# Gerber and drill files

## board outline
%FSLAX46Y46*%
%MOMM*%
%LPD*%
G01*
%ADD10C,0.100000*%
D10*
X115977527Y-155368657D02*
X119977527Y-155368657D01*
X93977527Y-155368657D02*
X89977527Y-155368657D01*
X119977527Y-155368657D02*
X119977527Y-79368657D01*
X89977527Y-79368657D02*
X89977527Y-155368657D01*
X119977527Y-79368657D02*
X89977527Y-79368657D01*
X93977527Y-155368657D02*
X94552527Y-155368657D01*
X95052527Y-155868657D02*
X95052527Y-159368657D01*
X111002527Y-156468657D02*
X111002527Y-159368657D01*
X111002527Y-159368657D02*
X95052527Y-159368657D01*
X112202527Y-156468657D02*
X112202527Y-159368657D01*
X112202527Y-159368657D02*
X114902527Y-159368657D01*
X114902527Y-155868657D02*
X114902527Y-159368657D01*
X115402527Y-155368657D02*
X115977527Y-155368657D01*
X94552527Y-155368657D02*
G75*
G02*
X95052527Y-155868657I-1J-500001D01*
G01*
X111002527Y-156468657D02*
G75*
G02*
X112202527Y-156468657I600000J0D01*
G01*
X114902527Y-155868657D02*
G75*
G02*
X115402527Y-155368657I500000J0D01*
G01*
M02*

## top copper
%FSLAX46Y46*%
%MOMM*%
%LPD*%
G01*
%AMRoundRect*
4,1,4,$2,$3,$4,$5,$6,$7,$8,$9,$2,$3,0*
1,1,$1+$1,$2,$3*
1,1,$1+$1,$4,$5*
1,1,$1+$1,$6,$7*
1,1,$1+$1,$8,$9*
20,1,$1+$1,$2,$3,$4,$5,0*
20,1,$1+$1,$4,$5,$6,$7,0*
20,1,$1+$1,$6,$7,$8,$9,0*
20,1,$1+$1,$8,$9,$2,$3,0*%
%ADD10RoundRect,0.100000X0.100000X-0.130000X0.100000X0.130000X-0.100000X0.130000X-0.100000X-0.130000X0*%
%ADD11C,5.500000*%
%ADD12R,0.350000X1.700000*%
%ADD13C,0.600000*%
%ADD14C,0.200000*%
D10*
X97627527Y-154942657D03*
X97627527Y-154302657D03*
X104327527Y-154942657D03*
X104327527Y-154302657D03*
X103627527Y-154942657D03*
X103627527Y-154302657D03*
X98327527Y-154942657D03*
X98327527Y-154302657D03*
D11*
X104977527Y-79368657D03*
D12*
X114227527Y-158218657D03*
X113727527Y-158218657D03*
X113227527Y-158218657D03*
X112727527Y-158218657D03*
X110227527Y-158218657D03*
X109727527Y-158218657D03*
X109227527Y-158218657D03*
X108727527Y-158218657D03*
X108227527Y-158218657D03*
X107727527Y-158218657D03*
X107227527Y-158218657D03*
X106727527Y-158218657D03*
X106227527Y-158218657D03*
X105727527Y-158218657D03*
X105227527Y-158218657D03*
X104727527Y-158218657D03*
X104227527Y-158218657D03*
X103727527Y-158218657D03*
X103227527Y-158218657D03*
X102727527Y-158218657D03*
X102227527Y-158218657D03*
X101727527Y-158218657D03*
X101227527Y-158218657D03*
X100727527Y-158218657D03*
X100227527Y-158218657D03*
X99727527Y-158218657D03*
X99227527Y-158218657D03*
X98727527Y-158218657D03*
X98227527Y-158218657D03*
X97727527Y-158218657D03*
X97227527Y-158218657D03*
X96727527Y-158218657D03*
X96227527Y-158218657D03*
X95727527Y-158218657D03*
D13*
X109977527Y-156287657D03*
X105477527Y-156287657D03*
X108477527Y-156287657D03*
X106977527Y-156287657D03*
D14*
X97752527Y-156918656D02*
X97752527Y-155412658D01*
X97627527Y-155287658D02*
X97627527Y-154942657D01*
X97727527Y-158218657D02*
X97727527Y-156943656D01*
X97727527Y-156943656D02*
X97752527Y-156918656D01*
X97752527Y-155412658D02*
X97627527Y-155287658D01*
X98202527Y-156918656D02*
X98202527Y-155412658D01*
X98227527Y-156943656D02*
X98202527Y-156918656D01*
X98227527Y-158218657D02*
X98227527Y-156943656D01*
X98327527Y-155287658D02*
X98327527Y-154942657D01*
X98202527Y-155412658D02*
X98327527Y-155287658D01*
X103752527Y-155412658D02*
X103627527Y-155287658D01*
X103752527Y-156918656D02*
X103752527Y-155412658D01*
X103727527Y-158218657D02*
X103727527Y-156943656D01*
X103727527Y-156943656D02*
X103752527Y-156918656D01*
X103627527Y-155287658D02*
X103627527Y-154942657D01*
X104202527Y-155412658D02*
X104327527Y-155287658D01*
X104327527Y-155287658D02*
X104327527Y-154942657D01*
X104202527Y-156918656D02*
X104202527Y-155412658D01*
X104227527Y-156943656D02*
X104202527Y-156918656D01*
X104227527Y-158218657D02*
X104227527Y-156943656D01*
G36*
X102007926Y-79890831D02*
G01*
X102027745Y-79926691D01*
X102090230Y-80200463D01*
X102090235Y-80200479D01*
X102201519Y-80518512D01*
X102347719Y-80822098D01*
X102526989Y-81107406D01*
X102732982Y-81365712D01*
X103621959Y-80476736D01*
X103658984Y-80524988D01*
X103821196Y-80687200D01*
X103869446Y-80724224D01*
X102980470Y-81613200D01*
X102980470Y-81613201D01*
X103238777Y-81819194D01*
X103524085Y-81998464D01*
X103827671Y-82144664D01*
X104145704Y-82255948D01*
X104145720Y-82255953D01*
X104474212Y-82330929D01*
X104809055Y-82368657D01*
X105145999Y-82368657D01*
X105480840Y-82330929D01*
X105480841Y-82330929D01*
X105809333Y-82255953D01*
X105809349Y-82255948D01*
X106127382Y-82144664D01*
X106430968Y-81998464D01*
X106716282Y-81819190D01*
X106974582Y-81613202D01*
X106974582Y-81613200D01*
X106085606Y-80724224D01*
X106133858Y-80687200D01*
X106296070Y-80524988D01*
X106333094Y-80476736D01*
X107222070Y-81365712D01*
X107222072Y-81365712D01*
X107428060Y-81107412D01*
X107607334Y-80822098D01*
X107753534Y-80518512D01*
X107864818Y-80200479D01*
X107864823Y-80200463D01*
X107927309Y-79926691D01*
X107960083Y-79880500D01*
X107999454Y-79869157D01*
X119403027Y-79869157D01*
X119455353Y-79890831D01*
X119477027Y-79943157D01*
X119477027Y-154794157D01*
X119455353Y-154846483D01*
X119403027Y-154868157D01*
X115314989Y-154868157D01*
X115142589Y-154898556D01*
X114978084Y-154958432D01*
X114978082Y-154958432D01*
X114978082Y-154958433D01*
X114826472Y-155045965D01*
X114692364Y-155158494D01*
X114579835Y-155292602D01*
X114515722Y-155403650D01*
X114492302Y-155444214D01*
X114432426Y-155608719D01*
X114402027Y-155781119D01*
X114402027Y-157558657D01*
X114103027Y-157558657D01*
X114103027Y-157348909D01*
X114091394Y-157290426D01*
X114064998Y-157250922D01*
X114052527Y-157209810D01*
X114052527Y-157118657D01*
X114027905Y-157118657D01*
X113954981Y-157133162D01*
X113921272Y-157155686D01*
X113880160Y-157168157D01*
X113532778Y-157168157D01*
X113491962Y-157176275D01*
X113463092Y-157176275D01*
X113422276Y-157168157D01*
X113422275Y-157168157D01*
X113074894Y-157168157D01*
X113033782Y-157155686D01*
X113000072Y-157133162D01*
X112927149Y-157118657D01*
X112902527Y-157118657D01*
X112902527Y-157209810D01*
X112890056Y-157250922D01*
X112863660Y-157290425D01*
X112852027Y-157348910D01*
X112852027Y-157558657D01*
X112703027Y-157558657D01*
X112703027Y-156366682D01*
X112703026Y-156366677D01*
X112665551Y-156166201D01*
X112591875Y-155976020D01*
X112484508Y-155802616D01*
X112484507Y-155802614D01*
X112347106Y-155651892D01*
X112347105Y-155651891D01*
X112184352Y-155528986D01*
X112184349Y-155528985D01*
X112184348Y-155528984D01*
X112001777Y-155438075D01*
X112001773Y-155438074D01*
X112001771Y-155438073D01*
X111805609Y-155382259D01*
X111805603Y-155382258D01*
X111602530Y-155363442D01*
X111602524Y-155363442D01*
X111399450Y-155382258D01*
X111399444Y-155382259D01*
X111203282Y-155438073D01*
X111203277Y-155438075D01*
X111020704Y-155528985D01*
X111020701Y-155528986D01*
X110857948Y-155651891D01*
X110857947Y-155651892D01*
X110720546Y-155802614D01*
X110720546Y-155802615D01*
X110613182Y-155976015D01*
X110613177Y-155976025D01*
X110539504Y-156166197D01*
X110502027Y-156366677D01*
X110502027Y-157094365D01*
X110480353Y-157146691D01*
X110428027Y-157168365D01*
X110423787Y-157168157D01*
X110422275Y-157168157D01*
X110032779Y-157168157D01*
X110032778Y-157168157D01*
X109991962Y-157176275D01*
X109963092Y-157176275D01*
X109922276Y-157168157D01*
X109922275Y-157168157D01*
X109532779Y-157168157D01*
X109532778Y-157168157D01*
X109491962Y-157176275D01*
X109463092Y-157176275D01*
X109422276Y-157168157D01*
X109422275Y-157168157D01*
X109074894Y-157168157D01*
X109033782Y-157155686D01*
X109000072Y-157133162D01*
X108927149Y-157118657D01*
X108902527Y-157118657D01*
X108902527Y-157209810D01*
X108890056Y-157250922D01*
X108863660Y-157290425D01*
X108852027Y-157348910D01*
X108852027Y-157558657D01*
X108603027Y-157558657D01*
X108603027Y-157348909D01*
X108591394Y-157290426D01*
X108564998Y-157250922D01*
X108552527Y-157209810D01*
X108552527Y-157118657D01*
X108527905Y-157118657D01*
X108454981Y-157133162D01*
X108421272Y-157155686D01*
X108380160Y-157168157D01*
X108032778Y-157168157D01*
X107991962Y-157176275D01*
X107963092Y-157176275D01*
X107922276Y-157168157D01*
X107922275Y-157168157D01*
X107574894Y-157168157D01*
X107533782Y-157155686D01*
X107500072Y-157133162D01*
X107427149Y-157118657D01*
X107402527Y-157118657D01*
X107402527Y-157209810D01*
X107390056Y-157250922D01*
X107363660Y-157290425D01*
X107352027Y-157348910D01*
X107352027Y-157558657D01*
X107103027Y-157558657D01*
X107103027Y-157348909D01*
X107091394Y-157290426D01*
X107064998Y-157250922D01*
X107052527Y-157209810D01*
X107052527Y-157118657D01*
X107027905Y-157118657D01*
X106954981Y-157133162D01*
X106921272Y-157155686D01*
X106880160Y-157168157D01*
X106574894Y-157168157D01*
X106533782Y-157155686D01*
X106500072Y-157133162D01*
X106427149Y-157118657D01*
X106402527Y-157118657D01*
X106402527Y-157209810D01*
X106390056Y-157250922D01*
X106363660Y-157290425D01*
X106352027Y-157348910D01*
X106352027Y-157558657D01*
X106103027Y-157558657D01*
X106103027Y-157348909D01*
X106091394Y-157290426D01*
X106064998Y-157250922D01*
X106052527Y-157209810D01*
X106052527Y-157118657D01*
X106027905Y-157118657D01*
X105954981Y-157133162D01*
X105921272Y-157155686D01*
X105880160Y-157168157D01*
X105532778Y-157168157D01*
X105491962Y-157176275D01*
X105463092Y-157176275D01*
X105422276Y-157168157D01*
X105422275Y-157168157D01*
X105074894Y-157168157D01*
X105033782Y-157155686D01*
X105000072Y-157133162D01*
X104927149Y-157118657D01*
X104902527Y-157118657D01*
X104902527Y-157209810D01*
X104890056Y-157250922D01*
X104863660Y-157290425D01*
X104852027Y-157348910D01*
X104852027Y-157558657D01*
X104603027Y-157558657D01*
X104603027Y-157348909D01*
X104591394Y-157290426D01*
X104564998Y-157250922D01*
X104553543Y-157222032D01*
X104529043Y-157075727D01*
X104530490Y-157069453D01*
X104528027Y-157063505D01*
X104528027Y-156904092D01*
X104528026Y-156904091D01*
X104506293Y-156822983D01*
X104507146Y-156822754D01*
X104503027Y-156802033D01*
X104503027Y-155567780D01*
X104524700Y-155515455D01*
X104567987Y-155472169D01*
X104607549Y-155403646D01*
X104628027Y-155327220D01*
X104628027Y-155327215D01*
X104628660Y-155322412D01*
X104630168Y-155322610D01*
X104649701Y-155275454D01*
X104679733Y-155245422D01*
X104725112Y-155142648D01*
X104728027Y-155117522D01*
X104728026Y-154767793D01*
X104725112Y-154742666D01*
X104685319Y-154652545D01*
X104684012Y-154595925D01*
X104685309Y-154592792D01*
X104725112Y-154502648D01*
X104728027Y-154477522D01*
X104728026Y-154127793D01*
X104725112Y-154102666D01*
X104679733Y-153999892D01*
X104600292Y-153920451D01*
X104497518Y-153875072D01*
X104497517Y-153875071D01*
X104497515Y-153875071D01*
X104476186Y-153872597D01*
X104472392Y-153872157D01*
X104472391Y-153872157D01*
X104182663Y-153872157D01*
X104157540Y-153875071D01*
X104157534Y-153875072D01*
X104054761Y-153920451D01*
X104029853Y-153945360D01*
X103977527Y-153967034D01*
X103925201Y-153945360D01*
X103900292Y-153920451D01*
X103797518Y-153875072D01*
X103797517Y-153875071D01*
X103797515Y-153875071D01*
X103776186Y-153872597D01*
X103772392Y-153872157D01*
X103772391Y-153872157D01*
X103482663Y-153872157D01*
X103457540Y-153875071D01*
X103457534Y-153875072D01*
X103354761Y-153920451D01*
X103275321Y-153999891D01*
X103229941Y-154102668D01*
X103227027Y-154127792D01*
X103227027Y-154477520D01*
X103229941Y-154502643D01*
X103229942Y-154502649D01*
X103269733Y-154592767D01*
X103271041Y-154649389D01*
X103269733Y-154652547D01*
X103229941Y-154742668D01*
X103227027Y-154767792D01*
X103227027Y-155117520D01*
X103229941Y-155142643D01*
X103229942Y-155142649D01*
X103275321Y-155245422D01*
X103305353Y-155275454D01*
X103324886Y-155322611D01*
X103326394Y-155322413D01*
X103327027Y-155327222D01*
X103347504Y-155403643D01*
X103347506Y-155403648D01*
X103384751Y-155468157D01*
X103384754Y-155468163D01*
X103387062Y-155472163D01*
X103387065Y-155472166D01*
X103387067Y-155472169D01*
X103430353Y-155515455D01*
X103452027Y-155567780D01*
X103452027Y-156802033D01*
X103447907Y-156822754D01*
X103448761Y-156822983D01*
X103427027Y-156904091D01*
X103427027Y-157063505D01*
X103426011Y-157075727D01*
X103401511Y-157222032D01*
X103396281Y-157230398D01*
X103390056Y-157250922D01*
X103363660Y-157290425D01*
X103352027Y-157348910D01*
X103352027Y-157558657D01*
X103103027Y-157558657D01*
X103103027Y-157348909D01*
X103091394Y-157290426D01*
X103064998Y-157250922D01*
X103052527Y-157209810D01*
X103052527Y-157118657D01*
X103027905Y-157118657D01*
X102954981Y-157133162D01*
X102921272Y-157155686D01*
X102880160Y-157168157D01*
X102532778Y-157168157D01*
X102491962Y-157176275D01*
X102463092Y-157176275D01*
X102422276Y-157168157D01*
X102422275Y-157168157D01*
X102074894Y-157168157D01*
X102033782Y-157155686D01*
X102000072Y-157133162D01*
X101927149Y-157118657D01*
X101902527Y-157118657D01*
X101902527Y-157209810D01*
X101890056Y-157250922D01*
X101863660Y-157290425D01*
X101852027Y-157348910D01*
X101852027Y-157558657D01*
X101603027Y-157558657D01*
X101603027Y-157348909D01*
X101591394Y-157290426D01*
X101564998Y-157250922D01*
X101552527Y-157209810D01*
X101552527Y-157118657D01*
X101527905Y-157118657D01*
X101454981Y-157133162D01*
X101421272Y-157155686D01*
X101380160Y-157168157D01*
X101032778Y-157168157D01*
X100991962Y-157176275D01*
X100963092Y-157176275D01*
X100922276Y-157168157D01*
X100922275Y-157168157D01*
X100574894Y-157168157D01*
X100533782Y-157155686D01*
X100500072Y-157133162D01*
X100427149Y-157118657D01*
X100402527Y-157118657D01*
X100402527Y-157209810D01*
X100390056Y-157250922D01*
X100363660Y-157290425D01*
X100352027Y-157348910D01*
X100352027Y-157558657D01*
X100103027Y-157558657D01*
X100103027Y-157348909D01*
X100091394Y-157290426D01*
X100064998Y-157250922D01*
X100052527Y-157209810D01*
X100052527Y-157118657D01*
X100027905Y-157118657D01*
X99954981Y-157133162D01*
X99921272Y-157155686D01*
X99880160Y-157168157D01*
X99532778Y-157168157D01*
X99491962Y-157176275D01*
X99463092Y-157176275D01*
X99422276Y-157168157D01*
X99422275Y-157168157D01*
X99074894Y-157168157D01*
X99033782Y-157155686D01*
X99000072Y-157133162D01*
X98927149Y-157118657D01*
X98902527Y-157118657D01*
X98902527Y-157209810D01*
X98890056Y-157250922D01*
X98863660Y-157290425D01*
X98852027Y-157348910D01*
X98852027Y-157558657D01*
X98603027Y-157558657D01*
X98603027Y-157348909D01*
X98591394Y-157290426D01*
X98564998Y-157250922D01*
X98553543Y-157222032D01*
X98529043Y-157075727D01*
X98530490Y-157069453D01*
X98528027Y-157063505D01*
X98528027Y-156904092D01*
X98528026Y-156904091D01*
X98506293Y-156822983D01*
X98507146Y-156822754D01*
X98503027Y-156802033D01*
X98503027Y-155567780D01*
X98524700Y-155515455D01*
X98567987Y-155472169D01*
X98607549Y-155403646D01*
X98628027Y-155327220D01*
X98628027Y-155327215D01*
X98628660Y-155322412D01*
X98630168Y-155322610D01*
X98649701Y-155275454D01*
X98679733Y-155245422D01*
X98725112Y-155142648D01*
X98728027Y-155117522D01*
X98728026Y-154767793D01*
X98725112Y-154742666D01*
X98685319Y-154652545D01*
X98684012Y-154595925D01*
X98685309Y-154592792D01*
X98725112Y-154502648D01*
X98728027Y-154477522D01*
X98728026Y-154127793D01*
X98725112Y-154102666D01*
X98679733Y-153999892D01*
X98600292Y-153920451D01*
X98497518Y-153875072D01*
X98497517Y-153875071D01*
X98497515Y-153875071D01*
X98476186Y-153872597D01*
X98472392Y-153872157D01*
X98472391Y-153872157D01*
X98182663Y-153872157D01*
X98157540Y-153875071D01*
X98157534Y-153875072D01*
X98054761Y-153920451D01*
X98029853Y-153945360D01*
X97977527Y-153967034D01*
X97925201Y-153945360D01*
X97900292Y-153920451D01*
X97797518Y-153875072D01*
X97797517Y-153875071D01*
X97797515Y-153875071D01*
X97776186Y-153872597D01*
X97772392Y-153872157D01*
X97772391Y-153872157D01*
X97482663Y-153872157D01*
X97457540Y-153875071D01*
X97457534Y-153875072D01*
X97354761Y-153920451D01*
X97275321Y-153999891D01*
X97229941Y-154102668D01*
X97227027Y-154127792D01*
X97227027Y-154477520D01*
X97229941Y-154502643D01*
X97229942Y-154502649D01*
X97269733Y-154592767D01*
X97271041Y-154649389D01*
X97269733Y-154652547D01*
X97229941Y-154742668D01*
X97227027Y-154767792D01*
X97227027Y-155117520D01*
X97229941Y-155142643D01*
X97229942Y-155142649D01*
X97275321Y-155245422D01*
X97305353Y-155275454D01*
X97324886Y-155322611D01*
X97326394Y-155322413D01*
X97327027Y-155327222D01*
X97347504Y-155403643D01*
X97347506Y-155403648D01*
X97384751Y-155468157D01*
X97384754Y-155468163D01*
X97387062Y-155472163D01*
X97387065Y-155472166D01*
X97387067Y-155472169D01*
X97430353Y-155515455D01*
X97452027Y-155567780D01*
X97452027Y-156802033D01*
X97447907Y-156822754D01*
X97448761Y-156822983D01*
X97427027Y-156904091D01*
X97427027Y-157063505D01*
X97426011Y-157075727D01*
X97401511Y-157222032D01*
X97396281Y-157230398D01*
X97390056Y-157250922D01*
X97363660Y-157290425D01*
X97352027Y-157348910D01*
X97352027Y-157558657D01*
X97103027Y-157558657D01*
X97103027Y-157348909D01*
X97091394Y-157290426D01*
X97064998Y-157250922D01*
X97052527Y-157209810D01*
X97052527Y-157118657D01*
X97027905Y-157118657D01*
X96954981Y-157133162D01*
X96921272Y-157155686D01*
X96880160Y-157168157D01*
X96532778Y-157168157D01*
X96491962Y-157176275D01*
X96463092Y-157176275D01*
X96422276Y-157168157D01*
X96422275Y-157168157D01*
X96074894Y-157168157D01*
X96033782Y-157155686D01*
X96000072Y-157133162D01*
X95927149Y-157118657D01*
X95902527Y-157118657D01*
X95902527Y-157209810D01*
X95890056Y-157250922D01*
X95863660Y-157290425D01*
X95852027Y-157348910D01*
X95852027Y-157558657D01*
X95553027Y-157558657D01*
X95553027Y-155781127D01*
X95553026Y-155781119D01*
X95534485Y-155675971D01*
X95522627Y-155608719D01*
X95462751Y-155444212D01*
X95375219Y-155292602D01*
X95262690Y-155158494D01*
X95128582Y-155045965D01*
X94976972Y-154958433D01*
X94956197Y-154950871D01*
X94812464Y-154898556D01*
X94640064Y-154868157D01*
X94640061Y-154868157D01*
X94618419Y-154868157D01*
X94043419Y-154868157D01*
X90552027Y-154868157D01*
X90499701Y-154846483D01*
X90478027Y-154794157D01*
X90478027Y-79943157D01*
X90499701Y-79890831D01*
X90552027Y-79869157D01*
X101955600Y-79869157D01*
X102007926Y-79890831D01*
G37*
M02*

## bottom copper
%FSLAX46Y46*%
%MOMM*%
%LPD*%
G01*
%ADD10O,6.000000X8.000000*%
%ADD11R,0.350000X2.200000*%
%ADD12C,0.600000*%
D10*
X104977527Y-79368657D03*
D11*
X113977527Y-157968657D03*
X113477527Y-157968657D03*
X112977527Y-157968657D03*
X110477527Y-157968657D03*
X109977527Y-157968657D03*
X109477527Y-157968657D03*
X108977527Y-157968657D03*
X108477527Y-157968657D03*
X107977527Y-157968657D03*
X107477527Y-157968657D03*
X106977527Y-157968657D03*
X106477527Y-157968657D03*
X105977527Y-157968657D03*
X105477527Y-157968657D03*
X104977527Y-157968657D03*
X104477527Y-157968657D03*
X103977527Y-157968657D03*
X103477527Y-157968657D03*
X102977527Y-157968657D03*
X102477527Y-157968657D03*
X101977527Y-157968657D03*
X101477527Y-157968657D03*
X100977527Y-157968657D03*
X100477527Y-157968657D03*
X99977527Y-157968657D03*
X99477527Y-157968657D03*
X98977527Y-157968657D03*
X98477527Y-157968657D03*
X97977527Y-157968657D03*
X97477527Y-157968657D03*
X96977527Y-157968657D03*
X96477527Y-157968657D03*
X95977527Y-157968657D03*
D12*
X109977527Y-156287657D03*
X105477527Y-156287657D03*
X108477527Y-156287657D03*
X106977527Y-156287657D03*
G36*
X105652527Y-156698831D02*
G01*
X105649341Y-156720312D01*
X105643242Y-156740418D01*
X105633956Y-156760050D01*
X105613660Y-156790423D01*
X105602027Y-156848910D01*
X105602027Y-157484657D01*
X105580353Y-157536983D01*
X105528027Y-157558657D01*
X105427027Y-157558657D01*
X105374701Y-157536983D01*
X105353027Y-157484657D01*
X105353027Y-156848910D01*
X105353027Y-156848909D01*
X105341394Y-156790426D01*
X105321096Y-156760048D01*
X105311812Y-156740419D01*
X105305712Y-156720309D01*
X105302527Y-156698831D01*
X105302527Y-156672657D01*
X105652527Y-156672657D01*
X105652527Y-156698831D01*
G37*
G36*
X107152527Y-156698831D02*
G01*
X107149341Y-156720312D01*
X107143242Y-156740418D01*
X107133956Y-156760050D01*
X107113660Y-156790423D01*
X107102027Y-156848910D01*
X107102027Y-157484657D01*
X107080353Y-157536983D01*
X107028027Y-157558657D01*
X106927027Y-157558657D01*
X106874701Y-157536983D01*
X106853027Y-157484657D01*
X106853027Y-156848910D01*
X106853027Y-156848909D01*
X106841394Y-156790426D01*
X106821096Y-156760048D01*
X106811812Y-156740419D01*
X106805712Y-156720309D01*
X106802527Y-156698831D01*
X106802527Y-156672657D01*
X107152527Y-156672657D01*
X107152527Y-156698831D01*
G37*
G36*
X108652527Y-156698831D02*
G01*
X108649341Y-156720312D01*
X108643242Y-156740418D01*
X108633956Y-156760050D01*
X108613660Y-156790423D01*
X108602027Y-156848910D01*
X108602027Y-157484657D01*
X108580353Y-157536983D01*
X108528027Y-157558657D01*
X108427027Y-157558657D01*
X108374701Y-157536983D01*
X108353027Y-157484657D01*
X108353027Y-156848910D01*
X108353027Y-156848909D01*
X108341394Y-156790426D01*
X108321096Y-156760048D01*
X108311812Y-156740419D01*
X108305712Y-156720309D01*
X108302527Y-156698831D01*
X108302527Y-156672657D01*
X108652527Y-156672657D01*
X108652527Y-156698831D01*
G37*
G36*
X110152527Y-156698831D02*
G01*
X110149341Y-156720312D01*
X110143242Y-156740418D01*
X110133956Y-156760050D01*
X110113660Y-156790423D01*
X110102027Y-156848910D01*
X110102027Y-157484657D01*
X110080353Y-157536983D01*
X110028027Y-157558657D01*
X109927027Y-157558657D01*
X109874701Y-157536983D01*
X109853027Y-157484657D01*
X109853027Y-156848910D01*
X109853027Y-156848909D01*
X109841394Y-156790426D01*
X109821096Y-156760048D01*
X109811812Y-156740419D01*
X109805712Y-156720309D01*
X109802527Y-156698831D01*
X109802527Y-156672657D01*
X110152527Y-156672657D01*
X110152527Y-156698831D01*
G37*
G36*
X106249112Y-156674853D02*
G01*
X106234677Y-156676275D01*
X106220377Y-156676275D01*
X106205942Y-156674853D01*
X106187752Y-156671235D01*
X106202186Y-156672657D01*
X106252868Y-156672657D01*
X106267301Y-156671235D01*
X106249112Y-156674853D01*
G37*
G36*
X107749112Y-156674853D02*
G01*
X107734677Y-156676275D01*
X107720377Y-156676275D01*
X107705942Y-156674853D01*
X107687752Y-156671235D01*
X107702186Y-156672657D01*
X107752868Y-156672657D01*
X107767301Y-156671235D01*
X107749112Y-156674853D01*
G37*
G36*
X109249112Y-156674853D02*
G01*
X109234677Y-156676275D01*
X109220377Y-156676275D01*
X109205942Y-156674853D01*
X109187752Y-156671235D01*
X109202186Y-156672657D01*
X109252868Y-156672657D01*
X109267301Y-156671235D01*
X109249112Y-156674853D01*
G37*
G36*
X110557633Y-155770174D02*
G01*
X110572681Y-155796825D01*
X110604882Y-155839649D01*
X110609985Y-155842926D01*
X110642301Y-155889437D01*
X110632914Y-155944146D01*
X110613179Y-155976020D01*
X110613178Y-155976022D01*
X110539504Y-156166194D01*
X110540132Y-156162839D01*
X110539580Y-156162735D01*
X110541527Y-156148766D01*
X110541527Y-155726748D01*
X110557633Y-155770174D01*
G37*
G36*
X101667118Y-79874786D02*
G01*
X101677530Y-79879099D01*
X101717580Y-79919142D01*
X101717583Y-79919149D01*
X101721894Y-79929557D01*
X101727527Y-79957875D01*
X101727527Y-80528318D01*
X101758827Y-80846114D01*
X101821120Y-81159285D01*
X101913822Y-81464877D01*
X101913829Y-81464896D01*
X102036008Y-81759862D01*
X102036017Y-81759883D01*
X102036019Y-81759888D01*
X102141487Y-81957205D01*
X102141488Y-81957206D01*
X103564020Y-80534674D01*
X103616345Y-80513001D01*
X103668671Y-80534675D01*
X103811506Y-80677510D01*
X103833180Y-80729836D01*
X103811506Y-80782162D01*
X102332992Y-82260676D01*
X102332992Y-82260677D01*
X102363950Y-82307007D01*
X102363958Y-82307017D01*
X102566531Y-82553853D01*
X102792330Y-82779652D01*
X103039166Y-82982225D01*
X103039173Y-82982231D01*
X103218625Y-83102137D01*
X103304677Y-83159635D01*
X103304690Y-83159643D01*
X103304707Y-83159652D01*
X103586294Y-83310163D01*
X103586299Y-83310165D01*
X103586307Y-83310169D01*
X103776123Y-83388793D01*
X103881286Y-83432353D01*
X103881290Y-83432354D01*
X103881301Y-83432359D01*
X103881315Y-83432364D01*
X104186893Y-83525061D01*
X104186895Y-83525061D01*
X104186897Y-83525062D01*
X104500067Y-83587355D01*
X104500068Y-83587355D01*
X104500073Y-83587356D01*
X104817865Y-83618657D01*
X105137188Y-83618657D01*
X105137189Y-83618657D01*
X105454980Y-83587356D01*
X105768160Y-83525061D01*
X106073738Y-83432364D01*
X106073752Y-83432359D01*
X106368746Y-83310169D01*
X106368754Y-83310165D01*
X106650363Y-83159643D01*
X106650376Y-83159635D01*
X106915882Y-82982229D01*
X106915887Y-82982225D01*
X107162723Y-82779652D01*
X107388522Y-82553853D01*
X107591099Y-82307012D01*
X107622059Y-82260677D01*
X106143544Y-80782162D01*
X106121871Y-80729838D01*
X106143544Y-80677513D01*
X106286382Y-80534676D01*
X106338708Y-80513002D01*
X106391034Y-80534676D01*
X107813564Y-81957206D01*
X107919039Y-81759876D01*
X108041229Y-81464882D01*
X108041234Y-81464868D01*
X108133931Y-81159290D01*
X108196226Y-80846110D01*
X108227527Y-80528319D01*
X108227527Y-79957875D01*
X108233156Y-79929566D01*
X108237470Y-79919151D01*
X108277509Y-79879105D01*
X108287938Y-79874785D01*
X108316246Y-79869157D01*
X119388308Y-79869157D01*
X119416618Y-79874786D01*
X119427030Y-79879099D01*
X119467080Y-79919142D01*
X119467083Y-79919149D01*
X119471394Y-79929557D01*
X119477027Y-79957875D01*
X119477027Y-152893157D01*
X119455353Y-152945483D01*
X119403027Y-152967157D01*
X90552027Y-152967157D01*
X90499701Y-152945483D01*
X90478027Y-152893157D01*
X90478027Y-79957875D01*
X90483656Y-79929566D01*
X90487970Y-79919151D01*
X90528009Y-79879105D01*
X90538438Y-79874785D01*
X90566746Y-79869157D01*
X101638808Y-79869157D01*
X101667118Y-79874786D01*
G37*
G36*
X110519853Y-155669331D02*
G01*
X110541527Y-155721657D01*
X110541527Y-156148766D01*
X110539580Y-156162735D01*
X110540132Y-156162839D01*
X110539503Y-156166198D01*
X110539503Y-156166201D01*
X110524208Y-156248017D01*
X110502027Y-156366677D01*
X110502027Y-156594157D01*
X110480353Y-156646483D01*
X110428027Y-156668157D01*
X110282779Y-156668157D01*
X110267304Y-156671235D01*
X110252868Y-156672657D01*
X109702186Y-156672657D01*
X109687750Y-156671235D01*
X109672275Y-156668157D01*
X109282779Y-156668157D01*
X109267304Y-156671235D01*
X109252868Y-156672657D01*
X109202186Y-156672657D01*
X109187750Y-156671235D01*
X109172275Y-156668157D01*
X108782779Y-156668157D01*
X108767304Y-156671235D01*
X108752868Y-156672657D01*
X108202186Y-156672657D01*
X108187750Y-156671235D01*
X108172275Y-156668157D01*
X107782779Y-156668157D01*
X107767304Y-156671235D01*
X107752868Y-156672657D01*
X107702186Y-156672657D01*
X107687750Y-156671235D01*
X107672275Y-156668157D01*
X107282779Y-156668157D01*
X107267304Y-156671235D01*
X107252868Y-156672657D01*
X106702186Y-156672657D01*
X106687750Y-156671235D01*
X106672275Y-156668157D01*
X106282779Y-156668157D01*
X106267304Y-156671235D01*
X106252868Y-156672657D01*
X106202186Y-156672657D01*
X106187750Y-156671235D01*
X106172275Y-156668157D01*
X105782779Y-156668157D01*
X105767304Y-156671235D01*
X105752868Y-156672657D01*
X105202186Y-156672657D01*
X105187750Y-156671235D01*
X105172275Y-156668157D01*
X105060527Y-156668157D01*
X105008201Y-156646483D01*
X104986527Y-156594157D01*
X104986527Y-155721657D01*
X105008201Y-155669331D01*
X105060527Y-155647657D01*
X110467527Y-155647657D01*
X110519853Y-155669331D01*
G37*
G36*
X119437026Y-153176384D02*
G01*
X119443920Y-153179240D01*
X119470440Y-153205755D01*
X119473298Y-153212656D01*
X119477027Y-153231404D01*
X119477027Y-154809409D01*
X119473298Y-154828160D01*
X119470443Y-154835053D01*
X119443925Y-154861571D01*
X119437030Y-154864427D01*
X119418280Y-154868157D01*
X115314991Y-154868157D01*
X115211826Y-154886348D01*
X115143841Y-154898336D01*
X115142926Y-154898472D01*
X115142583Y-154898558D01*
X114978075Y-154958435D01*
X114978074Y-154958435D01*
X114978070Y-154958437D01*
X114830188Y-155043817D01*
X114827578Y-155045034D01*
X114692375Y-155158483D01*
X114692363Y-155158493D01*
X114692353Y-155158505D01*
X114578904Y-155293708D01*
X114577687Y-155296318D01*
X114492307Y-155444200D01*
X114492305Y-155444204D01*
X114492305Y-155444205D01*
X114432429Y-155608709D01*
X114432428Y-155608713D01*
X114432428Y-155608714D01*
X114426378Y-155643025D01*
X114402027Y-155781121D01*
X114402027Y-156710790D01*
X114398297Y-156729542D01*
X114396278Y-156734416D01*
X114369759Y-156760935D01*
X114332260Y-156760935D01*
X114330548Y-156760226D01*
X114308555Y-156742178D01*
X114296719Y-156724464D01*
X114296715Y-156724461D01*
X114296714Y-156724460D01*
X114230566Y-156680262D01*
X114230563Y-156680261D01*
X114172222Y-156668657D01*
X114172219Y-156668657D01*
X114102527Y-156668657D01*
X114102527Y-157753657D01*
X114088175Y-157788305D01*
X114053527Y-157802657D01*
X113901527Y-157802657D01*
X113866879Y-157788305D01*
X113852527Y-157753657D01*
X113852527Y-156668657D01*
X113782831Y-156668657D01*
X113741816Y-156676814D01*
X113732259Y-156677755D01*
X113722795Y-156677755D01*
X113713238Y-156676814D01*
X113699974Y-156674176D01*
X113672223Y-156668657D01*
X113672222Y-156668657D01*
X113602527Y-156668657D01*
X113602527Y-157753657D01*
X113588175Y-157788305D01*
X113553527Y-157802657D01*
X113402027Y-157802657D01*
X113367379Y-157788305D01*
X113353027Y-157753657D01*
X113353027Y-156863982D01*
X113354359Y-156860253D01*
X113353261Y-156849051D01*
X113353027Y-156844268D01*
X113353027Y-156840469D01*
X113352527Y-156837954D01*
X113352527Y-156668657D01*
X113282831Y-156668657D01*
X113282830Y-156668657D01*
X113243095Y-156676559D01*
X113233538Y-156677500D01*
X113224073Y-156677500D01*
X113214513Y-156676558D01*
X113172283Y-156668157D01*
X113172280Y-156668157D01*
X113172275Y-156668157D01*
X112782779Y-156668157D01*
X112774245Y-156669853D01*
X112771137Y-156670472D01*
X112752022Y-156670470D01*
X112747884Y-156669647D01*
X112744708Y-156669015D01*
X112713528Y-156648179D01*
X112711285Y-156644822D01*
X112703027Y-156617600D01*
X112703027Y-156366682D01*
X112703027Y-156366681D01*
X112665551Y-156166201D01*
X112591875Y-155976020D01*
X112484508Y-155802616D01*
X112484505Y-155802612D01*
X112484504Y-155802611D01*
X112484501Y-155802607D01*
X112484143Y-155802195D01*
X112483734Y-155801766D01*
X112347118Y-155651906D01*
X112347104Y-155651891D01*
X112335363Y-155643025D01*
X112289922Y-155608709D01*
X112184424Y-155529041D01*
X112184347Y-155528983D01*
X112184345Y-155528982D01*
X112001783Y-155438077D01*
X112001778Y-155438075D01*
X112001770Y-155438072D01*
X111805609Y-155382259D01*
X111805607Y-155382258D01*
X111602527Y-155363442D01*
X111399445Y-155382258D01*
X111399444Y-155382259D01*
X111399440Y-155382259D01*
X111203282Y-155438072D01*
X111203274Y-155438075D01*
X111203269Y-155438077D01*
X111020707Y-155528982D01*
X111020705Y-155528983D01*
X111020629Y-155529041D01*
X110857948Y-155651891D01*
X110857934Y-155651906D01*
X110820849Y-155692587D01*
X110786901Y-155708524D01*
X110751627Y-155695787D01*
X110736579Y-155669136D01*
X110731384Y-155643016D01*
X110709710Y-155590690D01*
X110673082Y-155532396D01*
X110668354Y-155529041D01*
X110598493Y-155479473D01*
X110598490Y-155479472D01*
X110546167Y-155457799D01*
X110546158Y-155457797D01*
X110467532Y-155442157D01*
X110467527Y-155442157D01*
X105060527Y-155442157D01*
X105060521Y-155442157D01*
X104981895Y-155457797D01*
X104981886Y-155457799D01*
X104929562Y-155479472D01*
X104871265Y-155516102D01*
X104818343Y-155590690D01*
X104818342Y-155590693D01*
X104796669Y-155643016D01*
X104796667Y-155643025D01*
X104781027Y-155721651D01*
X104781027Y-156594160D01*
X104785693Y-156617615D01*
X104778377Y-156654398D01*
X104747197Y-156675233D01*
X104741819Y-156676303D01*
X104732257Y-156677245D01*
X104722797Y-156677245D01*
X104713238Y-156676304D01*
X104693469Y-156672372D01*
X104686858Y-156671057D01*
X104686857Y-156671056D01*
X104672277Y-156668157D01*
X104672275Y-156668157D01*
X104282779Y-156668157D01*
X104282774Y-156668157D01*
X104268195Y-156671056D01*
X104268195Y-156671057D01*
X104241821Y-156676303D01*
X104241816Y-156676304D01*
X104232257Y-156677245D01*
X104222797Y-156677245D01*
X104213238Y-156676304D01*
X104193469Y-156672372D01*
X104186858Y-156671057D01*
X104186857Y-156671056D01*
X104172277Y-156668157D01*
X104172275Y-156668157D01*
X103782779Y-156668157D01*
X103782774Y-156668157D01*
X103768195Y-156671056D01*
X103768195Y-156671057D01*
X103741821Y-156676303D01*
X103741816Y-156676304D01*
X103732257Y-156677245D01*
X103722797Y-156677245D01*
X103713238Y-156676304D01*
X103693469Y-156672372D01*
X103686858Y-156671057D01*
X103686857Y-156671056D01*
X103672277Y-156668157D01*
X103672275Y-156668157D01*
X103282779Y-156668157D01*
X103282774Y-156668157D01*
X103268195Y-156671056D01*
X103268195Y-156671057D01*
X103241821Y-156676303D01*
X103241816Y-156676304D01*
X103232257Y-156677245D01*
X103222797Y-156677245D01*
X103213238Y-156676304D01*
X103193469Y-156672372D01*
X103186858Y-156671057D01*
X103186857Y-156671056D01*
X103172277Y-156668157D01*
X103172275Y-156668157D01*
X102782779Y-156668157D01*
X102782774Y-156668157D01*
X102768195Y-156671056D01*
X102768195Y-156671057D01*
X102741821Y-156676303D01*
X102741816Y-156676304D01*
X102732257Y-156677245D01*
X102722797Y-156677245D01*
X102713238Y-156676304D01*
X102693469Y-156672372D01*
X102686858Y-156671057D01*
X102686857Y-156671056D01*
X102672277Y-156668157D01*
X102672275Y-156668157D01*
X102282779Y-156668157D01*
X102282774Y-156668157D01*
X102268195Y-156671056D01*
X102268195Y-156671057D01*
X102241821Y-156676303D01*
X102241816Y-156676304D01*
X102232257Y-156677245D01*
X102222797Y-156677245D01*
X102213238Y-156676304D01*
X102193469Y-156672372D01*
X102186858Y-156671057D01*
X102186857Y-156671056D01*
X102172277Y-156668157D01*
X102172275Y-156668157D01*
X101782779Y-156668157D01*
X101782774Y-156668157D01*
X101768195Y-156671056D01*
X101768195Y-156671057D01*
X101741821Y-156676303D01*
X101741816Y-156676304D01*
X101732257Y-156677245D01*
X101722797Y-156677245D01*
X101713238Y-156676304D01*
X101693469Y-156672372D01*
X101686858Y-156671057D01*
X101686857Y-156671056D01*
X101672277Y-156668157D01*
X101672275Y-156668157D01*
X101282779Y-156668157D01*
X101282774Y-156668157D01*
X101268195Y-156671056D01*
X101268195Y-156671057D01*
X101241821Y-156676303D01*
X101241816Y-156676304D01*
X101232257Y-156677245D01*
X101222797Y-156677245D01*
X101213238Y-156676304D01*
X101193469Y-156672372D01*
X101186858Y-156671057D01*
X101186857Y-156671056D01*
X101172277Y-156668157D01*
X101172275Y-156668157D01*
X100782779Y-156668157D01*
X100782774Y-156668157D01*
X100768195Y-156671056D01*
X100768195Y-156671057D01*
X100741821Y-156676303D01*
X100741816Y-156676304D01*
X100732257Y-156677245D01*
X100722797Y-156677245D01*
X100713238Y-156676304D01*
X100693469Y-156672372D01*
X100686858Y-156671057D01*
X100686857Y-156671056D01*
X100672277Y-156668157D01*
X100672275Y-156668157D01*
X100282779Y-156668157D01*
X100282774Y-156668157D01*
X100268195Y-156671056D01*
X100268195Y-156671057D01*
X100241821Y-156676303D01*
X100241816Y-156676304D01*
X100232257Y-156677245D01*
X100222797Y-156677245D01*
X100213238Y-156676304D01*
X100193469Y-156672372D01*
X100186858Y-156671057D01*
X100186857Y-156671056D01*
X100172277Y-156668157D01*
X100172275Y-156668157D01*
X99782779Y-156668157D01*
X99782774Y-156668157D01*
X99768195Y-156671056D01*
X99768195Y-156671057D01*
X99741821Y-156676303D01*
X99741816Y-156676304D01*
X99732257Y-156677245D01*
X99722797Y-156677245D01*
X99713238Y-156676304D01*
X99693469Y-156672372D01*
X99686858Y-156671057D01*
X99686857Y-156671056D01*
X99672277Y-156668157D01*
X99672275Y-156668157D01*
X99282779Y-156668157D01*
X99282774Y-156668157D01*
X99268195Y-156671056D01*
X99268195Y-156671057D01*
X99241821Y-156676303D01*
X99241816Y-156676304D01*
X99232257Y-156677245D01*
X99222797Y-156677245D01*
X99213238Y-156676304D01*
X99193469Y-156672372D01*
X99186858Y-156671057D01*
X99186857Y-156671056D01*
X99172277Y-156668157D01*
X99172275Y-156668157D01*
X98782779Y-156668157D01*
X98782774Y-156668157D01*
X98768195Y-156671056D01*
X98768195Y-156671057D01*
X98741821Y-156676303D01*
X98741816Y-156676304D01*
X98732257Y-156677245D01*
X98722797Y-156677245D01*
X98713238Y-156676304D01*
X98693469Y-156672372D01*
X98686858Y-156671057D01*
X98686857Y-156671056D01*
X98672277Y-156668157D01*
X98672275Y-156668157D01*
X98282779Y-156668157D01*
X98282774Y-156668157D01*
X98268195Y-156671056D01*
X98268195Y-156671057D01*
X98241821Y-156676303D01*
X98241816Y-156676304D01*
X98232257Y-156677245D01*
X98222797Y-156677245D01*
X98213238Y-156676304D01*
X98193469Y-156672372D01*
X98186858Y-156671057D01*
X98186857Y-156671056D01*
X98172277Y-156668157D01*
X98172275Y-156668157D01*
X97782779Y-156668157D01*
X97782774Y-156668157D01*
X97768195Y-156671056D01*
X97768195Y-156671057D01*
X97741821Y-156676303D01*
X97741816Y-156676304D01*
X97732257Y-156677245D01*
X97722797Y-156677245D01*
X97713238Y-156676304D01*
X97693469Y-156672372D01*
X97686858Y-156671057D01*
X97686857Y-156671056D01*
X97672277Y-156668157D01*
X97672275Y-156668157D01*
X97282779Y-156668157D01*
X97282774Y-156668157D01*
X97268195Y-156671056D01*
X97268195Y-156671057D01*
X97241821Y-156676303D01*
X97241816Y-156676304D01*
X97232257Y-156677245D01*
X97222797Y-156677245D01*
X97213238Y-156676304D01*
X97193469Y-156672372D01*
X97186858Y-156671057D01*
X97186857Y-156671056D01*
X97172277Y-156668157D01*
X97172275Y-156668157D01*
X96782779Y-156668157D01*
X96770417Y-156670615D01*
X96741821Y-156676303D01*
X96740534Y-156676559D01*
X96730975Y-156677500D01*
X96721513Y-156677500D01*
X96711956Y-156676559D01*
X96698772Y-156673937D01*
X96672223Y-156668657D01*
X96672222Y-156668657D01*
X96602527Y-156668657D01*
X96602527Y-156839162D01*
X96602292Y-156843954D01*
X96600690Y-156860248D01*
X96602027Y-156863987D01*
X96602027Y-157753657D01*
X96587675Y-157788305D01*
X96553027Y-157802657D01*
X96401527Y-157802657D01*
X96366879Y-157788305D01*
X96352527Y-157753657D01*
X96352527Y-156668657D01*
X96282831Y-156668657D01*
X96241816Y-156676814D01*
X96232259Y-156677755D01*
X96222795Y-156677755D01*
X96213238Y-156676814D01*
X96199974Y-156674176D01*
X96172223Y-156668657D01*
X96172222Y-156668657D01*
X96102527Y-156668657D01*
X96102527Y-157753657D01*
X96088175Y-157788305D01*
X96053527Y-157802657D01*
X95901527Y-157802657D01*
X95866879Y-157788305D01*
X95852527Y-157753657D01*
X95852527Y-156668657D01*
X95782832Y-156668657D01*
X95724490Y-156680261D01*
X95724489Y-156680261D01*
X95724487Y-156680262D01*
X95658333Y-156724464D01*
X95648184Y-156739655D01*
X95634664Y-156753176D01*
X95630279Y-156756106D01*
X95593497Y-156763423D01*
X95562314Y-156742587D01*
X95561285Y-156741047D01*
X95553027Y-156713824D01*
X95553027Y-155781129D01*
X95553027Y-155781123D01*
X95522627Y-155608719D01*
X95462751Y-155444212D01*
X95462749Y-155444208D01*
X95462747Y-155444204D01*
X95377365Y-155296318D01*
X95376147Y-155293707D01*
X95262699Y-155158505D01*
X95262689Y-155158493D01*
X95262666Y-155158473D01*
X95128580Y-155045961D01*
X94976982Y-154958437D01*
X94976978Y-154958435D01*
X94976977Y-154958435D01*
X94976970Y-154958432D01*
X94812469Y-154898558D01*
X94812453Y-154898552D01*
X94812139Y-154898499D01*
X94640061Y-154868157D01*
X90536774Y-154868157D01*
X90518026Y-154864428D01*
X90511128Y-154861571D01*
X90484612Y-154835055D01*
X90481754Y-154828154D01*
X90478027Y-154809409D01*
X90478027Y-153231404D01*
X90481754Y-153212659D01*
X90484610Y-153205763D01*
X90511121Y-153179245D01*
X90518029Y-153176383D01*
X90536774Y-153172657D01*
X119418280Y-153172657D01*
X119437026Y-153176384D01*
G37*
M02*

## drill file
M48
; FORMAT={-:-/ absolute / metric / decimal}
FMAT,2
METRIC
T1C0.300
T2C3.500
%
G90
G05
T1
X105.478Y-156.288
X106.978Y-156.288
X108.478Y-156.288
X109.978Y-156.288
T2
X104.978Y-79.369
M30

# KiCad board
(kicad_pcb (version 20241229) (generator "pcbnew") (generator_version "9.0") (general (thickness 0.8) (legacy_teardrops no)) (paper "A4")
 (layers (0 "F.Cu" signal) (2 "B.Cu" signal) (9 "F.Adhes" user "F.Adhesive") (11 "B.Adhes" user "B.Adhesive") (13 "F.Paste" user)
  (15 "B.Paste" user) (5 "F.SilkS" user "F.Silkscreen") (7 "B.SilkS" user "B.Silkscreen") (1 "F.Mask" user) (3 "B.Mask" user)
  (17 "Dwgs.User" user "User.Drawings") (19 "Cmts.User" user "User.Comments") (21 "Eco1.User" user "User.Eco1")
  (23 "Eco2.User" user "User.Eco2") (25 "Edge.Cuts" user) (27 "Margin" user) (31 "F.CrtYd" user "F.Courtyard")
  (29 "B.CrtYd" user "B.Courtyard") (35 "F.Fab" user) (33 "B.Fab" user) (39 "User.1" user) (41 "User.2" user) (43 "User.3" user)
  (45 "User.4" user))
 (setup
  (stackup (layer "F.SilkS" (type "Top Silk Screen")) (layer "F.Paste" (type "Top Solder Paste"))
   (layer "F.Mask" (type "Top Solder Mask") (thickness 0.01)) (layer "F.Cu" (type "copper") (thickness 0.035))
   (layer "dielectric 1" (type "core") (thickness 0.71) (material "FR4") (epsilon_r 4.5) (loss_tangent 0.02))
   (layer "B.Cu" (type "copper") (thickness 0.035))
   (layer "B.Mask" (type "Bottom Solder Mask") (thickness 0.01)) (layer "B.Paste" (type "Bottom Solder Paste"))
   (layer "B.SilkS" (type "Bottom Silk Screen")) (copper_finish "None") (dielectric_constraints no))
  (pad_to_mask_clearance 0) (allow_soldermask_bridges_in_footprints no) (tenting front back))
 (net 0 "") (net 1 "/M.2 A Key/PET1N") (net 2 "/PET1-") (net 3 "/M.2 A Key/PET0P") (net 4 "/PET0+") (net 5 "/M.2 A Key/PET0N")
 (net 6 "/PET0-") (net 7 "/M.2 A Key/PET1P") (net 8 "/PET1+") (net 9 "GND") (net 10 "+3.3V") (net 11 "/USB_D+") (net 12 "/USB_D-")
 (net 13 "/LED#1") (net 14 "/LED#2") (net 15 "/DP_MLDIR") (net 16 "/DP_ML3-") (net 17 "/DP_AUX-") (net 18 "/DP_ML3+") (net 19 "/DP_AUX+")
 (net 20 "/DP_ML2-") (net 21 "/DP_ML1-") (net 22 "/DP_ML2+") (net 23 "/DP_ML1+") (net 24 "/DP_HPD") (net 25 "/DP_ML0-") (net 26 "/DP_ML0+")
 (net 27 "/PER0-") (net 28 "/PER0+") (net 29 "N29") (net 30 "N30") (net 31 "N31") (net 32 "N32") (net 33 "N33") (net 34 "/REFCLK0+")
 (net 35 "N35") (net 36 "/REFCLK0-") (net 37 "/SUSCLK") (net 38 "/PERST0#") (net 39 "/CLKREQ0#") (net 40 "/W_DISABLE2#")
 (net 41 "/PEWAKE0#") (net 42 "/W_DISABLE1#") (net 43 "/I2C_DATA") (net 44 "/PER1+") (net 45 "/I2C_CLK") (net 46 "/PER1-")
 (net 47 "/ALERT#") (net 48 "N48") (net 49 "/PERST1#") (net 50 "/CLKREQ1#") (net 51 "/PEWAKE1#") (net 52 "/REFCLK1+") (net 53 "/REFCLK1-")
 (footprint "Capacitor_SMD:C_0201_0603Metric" (layer "F.Cu") (at 97.627527 154.622657 90)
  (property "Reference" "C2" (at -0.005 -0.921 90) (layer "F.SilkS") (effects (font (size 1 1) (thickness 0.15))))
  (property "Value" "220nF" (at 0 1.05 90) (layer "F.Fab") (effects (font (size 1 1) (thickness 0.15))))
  (pad "" smd roundrect (at -0.345 0 90) (size 0.318 0.36) (layers "F.Paste") (roundrect_rratio 0.25))
  (pad "" smd roundrect (at 0.345 0 90) (size 0.318 0.36) (layers "F.Paste") (roundrect_rratio 0.25))
  (pad "1" smd roundrect (at -0.32 0 90) (size 0.46 0.4) (layers "F.Cu" "F.Mask") (roundrect_rratio 0.25) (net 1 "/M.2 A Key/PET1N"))
  (pad "2" smd roundrect (at 0.32 0 90) (size 0.46 0.4) (layers "F.Cu" "F.Mask") (roundrect_rratio 0.25) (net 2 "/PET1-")))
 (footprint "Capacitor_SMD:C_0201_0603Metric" (layer "F.Cu") (at 104.327527 154.622657 90)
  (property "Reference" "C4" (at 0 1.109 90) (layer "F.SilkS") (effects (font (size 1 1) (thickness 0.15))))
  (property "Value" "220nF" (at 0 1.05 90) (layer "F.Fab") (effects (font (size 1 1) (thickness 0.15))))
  (pad "" smd roundrect (at -0.345 0 90) (size 0.318 0.36) (layers "F.Paste") (roundrect_rratio 0.25))
  (pad "" smd roundrect (at 0.345 0 90) (size 0.318 0.36) (layers "F.Paste") (roundrect_rratio 0.25))
  (pad "1" smd roundrect (at -0.32 0 90) (size 0.46 0.4) (layers "F.Cu" "F.Mask") (roundrect_rratio 0.25) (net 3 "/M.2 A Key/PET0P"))
  (pad "2" smd roundrect (at 0.32 0 90) (size 0.46 0.4) (layers "F.Cu" "F.Mask") (roundrect_rratio 0.25) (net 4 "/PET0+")))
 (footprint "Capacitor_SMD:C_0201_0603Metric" (layer "F.Cu") (at 103.627527 154.622657 90)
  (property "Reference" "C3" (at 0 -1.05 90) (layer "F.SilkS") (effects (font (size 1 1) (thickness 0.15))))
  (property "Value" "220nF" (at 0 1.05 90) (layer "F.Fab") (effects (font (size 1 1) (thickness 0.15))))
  (pad "" smd roundrect (at -0.345 0 90) (size 0.318 0.36) (layers "F.Paste") (roundrect_rratio 0.25))
  (pad "" smd roundrect (at 0.345 0 90) (size 0.318 0.36) (layers "F.Paste") (roundrect_rratio 0.25))
  (pad "1" smd roundrect (at -0.32 0 90) (size 0.46 0.4) (layers "F.Cu" "F.Mask") (roundrect_rratio 0.25) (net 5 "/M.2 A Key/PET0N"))
  (pad "2" smd roundrect (at 0.32 0 90) (size 0.46 0.4) (layers "F.Cu" "F.Mask") (roundrect_rratio 0.25) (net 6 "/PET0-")))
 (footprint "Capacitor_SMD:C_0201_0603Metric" (layer "F.Cu") (at 98.327527 154.622657 90)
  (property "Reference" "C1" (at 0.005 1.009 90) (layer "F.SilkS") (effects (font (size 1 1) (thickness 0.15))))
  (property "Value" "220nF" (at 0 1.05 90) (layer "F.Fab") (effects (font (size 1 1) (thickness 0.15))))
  (pad "" smd roundrect (at -0.345 0 90) (size 0.318 0.36) (layers "F.Paste") (roundrect_rratio 0.25))
  (pad "" smd roundrect (at 0.345 0 90) (size 0.318 0.36) (layers "F.Paste") (roundrect_rratio 0.25))
  (pad "1" smd roundrect (at -0.32 0 90) (size 0.46 0.4) (layers "F.Cu" "F.Mask") (roundrect_rratio 0.25) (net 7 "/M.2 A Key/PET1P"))
  (pad "2" smd roundrect (at 0.32 0 90) (size 0.46 0.4) (layers "F.Cu" "F.Mask") (roundrect_rratio 0.25) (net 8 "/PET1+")))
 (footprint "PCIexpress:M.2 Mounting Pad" (layer "F.Cu") (at 104.977527 79.368657)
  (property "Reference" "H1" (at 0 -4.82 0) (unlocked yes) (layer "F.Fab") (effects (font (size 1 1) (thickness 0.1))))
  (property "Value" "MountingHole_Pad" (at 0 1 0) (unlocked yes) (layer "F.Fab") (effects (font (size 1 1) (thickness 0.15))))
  (pad "1" thru_hole circle (at 0 0) (size 5.5 5.5) (drill 3.5) (layers "*.Cu" "*.Mask") (remove_unused_layers no) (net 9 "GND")
   (padstack (mode front_inner_back)
    (layer "Inner" (shape circle) (size 5.5 5.5) (zone_connect -1))
    (layer "B.Cu" (shape oval) (size 6 8) (thermal_bridge_angle 45) (zone_connect -1)))))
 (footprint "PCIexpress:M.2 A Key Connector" (layer "F.Cu") (at 104.977527 158.258657)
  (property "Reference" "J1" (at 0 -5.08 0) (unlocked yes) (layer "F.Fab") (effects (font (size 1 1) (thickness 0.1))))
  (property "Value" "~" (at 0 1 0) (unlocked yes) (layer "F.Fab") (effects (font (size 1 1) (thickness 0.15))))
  (fp_line (start -11 -2.89) (end -10.425 -2.89) (stroke (width 0.1) (type default)) (layer "Edge.Cuts"))
  (fp_line (start -9.925 -2.39) (end -9.925 1.11) (stroke (width 0.1) (type default)) (layer "Edge.Cuts"))
  (fp_line (start 6.025 -1.79) (end 6.025 1.11) (stroke (width 0.1) (type default)) (layer "Edge.Cuts"))
  (fp_line (start 6.025 1.11) (end -9.925 1.11) (stroke (width 0.1) (type default)) (layer "Edge.Cuts"))
  (fp_line (start 7.225 -1.79) (end 7.225 1.11) (stroke (width 0.1) (type default)) (layer "Edge.Cuts"))
  (fp_line (start 7.225 1.11) (end 9.925 1.11) (stroke (width 0.1) (type default)) (layer "Edge.Cuts"))
  (fp_line (start 9.925 -2.39) (end 9.925 1.11) (stroke (width 0.1) (type default)) (layer "Edge.Cuts"))
  (fp_line (start 10.425 -2.89) (end 11 -2.89) (stroke (width 0.1) (type default)) (layer "Edge.Cuts"))
  (fp_arc (start -10.425 -2.89) (mid -10.071447 -2.743553) (end -9.925 -2.39) (stroke (width 0.1) (type default)) (layer "Edge.Cuts"))
  (fp_arc (start 6.025 -1.79) (mid 6.625 -2.39) (end 7.225 -1.79) (stroke (width 0.1) (type default)) (layer "Edge.Cuts"))
  (fp_arc (start 9.925 -2.39) (mid 10.071447 -2.743553) (end 10.425 -2.89) (stroke (width 0.1) (type default)) (layer "Edge.Cuts"))
  (pad "1" smd rect (at 9.25 -0.04 180) (size 0.35 1.7) (layers "F.Cu") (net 9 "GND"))
  (pad "2" smd rect (at 9 -0.29 180) (size 0.35 2.2) (layers "B.Cu") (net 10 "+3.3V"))
  (pad "3" smd rect (at 8.75 -0.04 180) (size 0.35 1.7) (layers "F.Cu") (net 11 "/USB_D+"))
  (pad "4" smd rect (at 8.5 -0.29 180) (size 0.35 2.2) (layers "B.Cu") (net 10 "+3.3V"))
  (pad "5" smd rect (at 8.25 -0.04 180) (size 0.35 1.7) (layers "F.Cu") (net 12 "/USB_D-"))
  (pad "6" smd rect (at 8 -0.29 180) (size 0.35 2.2) (layers "B.Cu") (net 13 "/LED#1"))
  (pad "7" smd rect (at 7.75 -0.04 180) (size 0.35 1.7) (layers "F.Cu") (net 9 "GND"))
  (pad "16" smd rect (at 5.5 -0.29 180) (size 0.35 2.2) (layers "B.Cu") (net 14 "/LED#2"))
  (pad "17" smd rect (at 5.25 -0.04 180) (size 0.35 1.7) (layers "F.Cu") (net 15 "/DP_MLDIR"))
  (pad "18" smd rect (at 5 -0.29 180) (size 0.35 2.2) (layers "B.Cu") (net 9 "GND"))
  (pad "19" smd rect (at 4.75 -0.04 180) (size 0.35 1.7) (layers "F.Cu") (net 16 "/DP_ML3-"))
  (pad "20" smd rect (at 4.5 -0.29 180) (size 0.35 2.2) (layers "B.Cu") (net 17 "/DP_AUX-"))
  (pad "21" smd rect (at 4.25 -0.04 180) (size 0.35 1.7) (layers "F.Cu") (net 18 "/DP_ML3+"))
  (pad "22" smd rect (at 4 -0.29 180) (size 0.35 2.2) (layers "B.Cu") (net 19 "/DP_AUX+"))
  (pad "23" smd rect (at 3.75 -0.04 180) (size 0.35 1.7) (layers "F.Cu") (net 9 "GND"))
  (pad "24" smd rect (at 3.5 -0.29 180) (size 0.35 2.2) (layers "B.Cu") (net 9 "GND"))
  (pad "25" smd rect (at 3.25 -0.04 180) (size 0.35 1.7) (layers "F.Cu") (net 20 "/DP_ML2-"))
  (pad "26" smd rect (at 3 -0.29 180) (size 0.35 2.2) (layers "B.Cu") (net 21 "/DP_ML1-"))
  (pad "27" smd rect (at 2.75 -0.04 180) (size 0.35 1.7) (layers "F.Cu") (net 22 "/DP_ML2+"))
  (pad "28" smd rect (at 2.5 -0.29 180) (size 0.35 2.2) (layers "B.Cu") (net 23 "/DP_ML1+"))
  (pad "29" smd rect (at 2.25 -0.04 180) (size 0.35 1.7) (layers "F.Cu") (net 9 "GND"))
  (pad "30" smd rect (at 2 -0.29 180) (size 0.35 2.2) (layers "B.Cu") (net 9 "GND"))
  (pad "31" smd rect (at 1.75 -0.04 180) (size 0.35 1.7) (layers "F.Cu") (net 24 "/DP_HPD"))
  (pad "32" smd rect (at 1.5 -0.29 180) (size 0.35 2.2) (layers "B.Cu") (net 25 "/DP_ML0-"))
  (pad "33" smd rect (at 1.25 -0.04 180) (size 0.35 1.7) (layers "F.Cu") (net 9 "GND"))
  (pad "34" smd rect (at 1 -0.29 180) (size 0.35 2.2) (layers "B.Cu") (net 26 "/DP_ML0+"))
  (pad "35" smd rect (at 0.75 -0.04 180) (size 0.35 1.7) (layers "F.Cu") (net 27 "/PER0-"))
  (pad "36" smd rect (at 0.5 -0.29 180) (size 0.35 2.2) (layers "B.Cu") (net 9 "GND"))
  (pad "37" smd rect (at 0.25 -0.04 180) (size 0.35 1.7) (layers "F.Cu") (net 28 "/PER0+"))
  (pad "38" smd rect (at 0 -0.29 180) (size 0.35 2.2) (layers "B.Cu") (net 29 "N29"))
  (pad "39" smd rect (at -0.25 -0.04 180) (size 0.35 1.7) (layers "F.Cu") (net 9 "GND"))
  (pad "40" smd rect (at -0.5 -0.29 180) (size 0.35 2.2) (layers "B.Cu") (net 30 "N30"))
  (pad "41" smd rect (at -0.75 -0.04 180) (size 0.35 1.7) (layers "F.Cu") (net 3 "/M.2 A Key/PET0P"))
  (pad "42" smd rect (at -1 -0.29 180) (size 0.35 2.2) (layers "B.Cu") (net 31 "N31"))
  (pad "43" smd rect (at -1.25 -0.04 180) (size 0.35 1.7) (layers "F.Cu") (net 5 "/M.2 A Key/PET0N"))
  (pad "44" smd rect (at -1.5 -0.29 180) (size 0.35 2.2) (layers "B.Cu") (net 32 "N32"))
  (pad "45" smd rect (at -1.75 -0.04 180) (size 0.35 1.7) (layers "F.Cu") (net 9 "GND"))
  (pad "46" smd rect (at -2 -0.29 180) (size 0.35 2.2) (layers "B.Cu") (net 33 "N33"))
  (pad "47" smd rect (at -2.25 -0.04 180) (size 0.35 1.7) (layers "F.Cu") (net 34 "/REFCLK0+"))
  (pad "48" smd rect (at -2.5 -0.29 180) (size 0.35 2.2) (layers "B.Cu") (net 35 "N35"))
  (pad "49" smd rect (at -2.75 -0.04 180) (size 0.35 1.7) (layers "F.Cu") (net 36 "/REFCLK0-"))
  (pad "50" smd rect (at -3 -0.29 180) (size 0.35 2.2) (layers "B.Cu") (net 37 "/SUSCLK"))
  (pad "51" smd rect (at -3.25 -0.04 180) (size 0.35 1.7) (layers "F.Cu") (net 9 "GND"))
  (pad "52" smd rect (at -3.5 -0.29 180) (size 0.35 2.2) (layers "B.Cu") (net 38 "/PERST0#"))
  (pad "53" smd rect (at -3.75 -0.04 180) (size 0.35 1.7) (layers "F.Cu") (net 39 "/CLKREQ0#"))
  (pad "54" smd rect (at -4 -0.29 180) (size 0.35 2.2) (layers "B.Cu") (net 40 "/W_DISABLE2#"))
  (pad "55" smd rect (at -4.25 -0.04 180) (size 0.35 1.7) (layers "F.Cu") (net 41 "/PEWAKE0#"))
  (pad "56" smd rect (at -4.5 -0.29 180) (size 0.35 2.2) (layers "B.Cu") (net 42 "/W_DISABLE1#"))
  (pad "57" smd rect (at -4.75 -0.04 180) (size 0.35 1.7) (layers "F.Cu") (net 9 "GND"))
  (pad "58" smd rect (at -5 -0.29 180) (size 0.35 2.2) (layers "B.Cu") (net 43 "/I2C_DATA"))
  (pad "59" smd rect (at -5.25 -0.04 180) (size 0.35 1.7) (layers "F.Cu") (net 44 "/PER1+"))
  (pad "60" smd rect (at -5.5 -0.29 180) (size 0.35 2.2) (layers "B.Cu") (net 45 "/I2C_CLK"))
  (pad "61" smd rect (at -5.75 -0.04 180) (size 0.35 1.7) (layers "F.Cu") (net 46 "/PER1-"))
  (pad "62" smd rect (at -6 -0.29 180) (size 0.35 2.2) (layers "B.Cu") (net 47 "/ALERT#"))
  (pad "63" smd rect (at -6.25 -0.04 180) (size 0.35 1.7) (layers "F.Cu") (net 9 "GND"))
  (pad "64" smd rect (at -6.5 -0.29 180) (size 0.35 2.2) (layers "B.Cu") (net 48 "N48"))
  (pad "65" smd rect (at -6.75 -0.04 180) (size 0.35 1.7) (layers "F.Cu") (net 7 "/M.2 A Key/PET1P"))
  (pad "66" smd rect (at -7 -0.29 180) (size 0.35 2.2) (layers "B.Cu") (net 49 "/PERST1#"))
  (pad "67" smd rect (at -7.25 -0.04 180) (size 0.35 1.7) (layers "F.Cu") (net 1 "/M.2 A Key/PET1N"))
  (pad "68" smd rect (at -7.5 -0.29 180) (size 0.35 2.2) (layers "B.Cu") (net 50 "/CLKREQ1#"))
  (pad "69" smd rect (at -7.75 -0.04 180) (size 0.35 1.7) (layers "F.Cu") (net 9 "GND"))
  (pad "70" smd rect (at -8 -0.29 180) (size 0.35 2.2) (layers "B.Cu") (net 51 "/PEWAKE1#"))
  (pad "71" smd rect (at -8.25 -0.04 180) (size 0.35 1.7) (layers "F.Cu") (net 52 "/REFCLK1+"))
  (pad "72" smd rect (at -8.5 -0.29 180) (size 0.35 2.2) (layers "B.Cu") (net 10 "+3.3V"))
  (pad "73" smd rect (at -8.75 -0.04 180) (size 0.35 1.7) (layers "F.Cu") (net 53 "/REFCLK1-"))
  (pad "74" smd rect (at -9 -0.29 180) (size 0.35 2.2) (layers "B.Cu") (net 10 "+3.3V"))
  (pad "75" smd rect (at -9.25 -0.04 180) (size 0.35 1.7) (layers "F.Cu") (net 9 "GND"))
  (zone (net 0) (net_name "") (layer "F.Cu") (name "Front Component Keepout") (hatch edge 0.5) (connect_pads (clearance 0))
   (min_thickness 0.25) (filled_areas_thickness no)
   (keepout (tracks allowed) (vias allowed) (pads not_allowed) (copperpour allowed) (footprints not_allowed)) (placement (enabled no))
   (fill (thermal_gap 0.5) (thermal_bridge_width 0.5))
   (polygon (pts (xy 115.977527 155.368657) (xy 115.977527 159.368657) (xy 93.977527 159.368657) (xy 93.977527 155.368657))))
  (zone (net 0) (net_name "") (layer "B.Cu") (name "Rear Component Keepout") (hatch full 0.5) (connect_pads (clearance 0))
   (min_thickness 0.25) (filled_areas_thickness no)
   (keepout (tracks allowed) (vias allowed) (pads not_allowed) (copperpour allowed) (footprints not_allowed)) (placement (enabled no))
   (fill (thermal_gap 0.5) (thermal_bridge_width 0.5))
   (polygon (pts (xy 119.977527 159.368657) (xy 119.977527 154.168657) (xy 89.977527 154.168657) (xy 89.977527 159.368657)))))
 (gr_line (start 115.977527 155.368657) (end 119.977527 155.368657) (stroke (width 0.1) (type default)) (layer "Edge.Cuts"))
 (gr_line (start 93.977527 155.368657) (end 89.977527 155.368657) (stroke (width 0.1) (type default)) (layer "Edge.Cuts"))
 (gr_line (start 119.977527 155.368657) (end 119.977527 79.368657) (stroke (width 0.1) (type default)) (layer "Edge.Cuts"))
 (gr_line (start 89.977527 79.368657) (end 89.977527 155.368657) (stroke (width 0.1) (type default)) (layer "Edge.Cuts"))
 (gr_line (start 119.977527 79.368657) (end 89.977527 79.368657) (stroke (width 0.1) (type solid)) (layer "Edge.Cuts"))
 (via (at 109.977527 156.287657) (size 0.6) (drill 0.3) (layers "F.Cu" "B.Cu") (free yes) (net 9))
 (via (at 105.477527 156.287657) (size 0.6) (drill 0.3) (layers "F.Cu" "B.Cu") (free yes) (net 9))
 (via (at 108.477527 156.287657) (size 0.6) (drill 0.3) (layers "F.Cu" "B.Cu") (free yes) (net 9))
 (via (at 106.977527 156.287657) (size 0.6) (drill 0.3) (layers "F.Cu" "B.Cu") (free yes) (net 9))
 (segment (start 97.752527 156.918656) (end 97.752527 155.412658) (width 0.2) (layer "F.Cu") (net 1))
 (segment (start 97.627527 155.287658) (end 97.627527 154.942657) (width 0.2) (layer "F.Cu") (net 1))
 (segment (start 97.727527 158.218657) (end 97.727527 156.943656) (width 0.2) (layer "F.Cu") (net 1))
 (segment (start 97.727527 156.943656) (end 97.752527 156.918656) (width 0.2) (layer "F.Cu") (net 1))
 (segment (start 97.752527 155.412658) (end 97.627527 155.287658) (width 0.2) (layer "F.Cu") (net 1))
 (segment (start 98.202527 156.918656) (end 98.202527 155.412658) (width 0.2) (layer "F.Cu") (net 7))
 (segment (start 98.227527 156.943656) (end 98.202527 156.918656) (width 0.2) (layer "F.Cu") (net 7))
 (segment (start 98.227527 158.218657) (end 98.227527 156.943656) (width 0.2) (layer "F.Cu") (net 7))
 (segment (start 98.327527 155.287658) (end 98.327527 154.942657) (width 0.2) (layer "F.Cu") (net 7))
 (segment (start 98.202527 155.412658) (end 98.327527 155.287658) (width 0.2) (layer "F.Cu") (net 7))
 (segment (start 103.752527 155.412658) (end 103.627527 155.287658) (width 0.2) (layer "F.Cu") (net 5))
 (segment (start 103.752527 156.918656) (end 103.752527 155.412658) (width 0.2) (layer "F.Cu") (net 5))
 (segment (start 103.727527 158.218657) (end 103.727527 156.943656) (width 0.2) (layer "F.Cu") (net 5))
 (segment (start 103.727527 156.943656) (end 103.752527 156.918656) (width 0.2) (layer "F.Cu") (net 5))
 (segment (start 103.627527 155.287658) (end 103.627527 154.942657) (width 0.2) (layer "F.Cu") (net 5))
 (segment (start 104.202527 155.412658) (end 104.327527 155.287658) (width 0.2) (layer "F.Cu") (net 3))
 (segment (start 104.327527 155.287658) (end 104.327527 154.942657) (width 0.2) (layer "F.Cu") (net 3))
 (segment (start 104.202527 156.918656) (end 104.202527 155.412658) (width 0.2) (layer "F.Cu") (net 3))
 (segment (start 104.227527 156.943656) (end 104.202527 156.918656) (width 0.2) (layer "F.Cu") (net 3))
 (segment (start 104.227527 158.218657) (end 104.227527 156.943656) (width 0.2) (layer "F.Cu") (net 3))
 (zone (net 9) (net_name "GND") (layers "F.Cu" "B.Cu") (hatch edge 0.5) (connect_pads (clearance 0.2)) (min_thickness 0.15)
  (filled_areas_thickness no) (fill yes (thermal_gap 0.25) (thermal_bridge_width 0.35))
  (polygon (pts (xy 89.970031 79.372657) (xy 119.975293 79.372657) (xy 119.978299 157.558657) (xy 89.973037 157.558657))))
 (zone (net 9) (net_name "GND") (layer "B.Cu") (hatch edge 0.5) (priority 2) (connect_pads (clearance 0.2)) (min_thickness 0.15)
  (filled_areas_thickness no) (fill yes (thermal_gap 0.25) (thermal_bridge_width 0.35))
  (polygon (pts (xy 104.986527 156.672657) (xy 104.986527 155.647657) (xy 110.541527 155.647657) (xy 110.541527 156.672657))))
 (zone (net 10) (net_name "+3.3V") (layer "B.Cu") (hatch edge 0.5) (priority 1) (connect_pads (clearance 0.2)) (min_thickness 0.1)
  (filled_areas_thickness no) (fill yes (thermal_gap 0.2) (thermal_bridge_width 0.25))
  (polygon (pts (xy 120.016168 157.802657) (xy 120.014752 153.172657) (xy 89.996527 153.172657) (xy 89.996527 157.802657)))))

